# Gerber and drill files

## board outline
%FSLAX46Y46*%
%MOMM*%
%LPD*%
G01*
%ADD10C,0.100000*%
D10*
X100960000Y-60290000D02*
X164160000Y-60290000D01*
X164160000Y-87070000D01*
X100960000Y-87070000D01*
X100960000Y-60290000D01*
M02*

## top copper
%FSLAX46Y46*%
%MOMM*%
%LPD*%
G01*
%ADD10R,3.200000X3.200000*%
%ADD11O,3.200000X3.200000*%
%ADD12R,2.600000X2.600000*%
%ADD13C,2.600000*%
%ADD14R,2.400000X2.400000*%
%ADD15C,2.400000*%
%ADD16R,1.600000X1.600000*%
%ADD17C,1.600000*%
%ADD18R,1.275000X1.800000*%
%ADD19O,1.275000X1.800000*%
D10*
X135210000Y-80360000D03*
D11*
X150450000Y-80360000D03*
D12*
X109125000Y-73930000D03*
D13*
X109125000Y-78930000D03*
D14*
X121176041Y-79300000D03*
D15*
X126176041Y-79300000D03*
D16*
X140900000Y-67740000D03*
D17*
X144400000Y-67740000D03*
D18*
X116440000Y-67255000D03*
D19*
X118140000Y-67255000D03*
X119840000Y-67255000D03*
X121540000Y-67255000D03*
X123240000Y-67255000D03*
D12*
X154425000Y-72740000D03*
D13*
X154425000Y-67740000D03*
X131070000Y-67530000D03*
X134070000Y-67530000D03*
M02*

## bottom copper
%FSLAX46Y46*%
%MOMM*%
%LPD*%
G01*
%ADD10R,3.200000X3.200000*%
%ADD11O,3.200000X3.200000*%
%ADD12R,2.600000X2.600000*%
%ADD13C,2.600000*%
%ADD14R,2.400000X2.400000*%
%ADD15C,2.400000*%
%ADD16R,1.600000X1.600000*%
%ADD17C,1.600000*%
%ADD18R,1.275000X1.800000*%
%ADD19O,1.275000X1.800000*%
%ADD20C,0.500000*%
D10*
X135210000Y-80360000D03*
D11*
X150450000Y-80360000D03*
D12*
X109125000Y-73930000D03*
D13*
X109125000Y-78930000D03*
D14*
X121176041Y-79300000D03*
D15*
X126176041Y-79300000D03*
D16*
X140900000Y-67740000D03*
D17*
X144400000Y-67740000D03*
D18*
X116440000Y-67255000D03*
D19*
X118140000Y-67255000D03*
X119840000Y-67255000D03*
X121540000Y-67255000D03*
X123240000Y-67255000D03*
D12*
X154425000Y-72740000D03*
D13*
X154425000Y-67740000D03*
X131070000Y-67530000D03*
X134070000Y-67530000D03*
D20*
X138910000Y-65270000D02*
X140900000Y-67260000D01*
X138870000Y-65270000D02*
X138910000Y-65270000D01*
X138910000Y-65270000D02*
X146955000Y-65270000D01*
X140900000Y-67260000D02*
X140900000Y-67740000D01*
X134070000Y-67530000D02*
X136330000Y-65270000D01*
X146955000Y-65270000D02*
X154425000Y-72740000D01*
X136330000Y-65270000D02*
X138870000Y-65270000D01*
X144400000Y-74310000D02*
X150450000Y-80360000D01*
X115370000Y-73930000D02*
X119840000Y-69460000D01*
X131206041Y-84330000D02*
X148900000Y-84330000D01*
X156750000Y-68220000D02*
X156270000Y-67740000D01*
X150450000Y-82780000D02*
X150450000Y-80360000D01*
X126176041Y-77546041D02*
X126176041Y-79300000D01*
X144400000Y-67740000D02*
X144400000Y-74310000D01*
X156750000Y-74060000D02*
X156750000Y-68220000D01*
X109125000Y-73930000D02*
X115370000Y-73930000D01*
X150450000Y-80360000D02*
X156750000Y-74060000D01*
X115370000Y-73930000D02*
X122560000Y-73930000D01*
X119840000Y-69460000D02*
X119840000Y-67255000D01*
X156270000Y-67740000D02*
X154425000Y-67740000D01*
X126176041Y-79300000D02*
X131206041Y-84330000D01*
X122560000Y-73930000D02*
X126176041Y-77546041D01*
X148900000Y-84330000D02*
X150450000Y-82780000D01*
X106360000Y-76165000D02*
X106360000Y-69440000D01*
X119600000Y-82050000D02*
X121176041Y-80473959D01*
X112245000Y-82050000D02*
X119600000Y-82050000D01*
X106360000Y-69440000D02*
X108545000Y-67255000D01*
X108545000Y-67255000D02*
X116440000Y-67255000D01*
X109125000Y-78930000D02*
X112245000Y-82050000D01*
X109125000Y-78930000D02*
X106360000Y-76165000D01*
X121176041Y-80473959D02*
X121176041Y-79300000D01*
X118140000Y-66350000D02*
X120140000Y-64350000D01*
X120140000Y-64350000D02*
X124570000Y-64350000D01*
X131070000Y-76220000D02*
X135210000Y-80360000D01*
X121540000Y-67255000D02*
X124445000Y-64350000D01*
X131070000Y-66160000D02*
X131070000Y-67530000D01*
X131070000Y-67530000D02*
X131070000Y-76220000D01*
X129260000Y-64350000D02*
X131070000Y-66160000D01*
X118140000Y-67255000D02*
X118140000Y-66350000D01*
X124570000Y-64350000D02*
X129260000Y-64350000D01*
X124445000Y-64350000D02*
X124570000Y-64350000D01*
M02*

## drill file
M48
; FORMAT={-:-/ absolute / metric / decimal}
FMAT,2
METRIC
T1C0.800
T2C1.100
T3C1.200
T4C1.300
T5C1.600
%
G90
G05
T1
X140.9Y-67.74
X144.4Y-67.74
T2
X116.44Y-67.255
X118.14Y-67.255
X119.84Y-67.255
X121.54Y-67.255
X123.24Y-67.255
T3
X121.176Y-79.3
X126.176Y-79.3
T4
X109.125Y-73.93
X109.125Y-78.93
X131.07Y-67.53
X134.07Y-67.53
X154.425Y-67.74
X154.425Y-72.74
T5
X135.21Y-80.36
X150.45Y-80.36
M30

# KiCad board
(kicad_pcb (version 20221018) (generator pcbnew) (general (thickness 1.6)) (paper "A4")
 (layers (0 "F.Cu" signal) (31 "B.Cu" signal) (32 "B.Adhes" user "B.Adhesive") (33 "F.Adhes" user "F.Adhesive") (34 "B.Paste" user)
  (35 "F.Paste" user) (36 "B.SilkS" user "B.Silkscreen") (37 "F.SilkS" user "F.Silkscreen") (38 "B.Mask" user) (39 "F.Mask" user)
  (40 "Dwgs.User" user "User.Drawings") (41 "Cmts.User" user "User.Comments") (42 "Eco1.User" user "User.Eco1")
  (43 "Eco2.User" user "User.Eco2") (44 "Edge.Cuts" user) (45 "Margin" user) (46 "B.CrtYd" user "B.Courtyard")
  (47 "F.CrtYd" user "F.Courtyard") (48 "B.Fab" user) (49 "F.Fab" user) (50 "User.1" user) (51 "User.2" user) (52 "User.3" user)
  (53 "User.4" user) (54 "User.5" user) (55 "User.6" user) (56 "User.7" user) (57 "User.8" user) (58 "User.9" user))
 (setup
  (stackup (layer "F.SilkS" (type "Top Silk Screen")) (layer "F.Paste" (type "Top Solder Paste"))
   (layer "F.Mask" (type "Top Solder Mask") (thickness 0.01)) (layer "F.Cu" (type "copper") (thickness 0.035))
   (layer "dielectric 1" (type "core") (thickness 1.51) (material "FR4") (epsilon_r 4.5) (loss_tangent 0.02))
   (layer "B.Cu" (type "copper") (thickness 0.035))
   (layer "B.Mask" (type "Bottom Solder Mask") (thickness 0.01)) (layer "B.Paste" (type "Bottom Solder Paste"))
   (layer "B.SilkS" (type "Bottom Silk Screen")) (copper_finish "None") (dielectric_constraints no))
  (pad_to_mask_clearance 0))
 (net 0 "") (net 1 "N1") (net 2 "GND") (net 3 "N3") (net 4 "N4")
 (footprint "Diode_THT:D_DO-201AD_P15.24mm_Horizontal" (layer "F.Cu") (at 135.21 80.36)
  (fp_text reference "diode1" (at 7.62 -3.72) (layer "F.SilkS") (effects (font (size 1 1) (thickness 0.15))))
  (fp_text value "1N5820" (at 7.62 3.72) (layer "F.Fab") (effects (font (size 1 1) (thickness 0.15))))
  (pad "1" thru_hole rect (at 0 0) (size 3.2 3.2) (drill 1.6) (layers "*.Cu" "*.Mask") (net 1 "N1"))
  (pad "2" thru_hole oval (at 15.24 0) (size 3.2 3.2) (drill 1.6) (layers "*.Cu" "*.Mask") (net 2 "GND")))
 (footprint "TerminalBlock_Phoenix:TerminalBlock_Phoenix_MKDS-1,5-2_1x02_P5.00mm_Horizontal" (layer "F.Cu") (at 109.125 73.93 -90)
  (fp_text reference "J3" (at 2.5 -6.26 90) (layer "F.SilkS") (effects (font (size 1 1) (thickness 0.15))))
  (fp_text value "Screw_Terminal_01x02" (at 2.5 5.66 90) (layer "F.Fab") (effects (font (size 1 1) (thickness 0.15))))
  (pad "1" thru_hole rect (at 0 0 270) (size 2.6 2.6) (drill 1.3) (layers "*.Cu" "*.Mask") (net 2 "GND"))
  (pad "2" thru_hole circle (at 5 0 270) (size 2.6 2.6) (drill 1.3) (layers "*.Cu" "*.Mask") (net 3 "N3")))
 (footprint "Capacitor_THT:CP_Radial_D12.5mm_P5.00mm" (layer "F.Cu") (at 121.176041 79.3)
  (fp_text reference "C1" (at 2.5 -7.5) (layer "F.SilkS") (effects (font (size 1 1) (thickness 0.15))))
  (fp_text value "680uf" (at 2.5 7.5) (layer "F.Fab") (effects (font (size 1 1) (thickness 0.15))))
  (pad "1" thru_hole rect (at 0 0) (size 2.4 2.4) (drill 1.2) (layers "*.Cu" "*.Mask") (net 3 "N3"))
  (pad "2" thru_hole circle (at 5 0) (size 2.4 2.4) (drill 1.2) (layers "*.Cu" "*.Mask") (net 2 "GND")))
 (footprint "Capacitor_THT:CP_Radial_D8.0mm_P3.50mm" (layer "F.Cu") (at 140.9 67.74)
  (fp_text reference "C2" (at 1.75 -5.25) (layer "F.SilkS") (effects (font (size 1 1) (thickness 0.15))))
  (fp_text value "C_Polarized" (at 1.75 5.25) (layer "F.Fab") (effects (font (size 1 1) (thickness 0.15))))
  (pad "1" thru_hole rect (at 0 0) (size 1.6 1.6) (drill 0.8) (layers "*.Cu" "*.Mask") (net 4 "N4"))
  (pad "2" thru_hole circle (at 3.5 0) (size 1.6 1.6) (drill 0.8) (layers "*.Cu" "*.Mask") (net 2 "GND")))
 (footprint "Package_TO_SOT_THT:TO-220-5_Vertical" (layer "F.Cu") (at 116.44 67.255)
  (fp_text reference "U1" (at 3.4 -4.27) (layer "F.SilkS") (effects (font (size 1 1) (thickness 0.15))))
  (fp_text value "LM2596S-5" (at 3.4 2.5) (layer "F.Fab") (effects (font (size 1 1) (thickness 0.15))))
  (pad "1" thru_hole rect (at 0 0) (size 1.275 1.8) (drill 1.1) (layers "*.Cu" "*.Mask") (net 3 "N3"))
  (pad "2" thru_hole oval (at 1.7 0) (size 1.275 1.8) (drill 1.1) (layers "*.Cu" "*.Mask") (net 1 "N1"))
  (pad "3" thru_hole oval (at 3.4 0) (size 1.275 1.8) (drill 1.1) (layers "*.Cu" "*.Mask") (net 2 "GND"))
  (pad "4" thru_hole oval (at 5.1 0) (size 1.275 1.8) (drill 1.1) (layers "*.Cu" "*.Mask") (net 1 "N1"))
  (pad "5" thru_hole oval (at 6.8 0) (size 1.275 1.8) (drill 1.1) (layers "*.Cu" "*.Mask") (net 2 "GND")))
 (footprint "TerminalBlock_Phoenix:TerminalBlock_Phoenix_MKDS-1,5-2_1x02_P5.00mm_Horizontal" (layer "F.Cu") (at 154.425 72.74 90)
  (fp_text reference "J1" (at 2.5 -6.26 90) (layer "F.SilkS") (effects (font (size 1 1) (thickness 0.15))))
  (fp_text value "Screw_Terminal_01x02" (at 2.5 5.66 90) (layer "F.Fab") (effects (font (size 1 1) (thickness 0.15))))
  (pad "1" thru_hole rect (at 0 0 90) (size 2.6 2.6) (drill 1.3) (layers "*.Cu" "*.Mask") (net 4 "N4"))
  (pad "2" thru_hole circle (at 5 0 90) (size 2.6 2.6) (drill 1.3) (layers "*.Cu" "*.Mask") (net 2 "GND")))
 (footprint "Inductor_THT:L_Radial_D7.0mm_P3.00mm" (layer "F.Cu") (at 131.07 67.53)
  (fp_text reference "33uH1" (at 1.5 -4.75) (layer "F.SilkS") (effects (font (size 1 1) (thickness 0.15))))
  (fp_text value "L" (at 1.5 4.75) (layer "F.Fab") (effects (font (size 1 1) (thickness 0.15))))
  (pad "1" thru_hole circle (at 0 0) (size 2.6 2.6) (drill 1.3) (layers "*.Cu" "*.Mask") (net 1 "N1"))
  (pad "2" thru_hole circle (at 3 0) (size 2.6 2.6) (drill 1.3) (layers "*.Cu" "*.Mask") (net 4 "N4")))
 (gr_rect (start 100.96 60.29) (end 164.16 87.07) (stroke (width 0.1) (type default)) (fill none) (layer "Edge.Cuts"))
 (segment (start 138.91 65.27) (end 140.9 67.26) (width 0.5) (layer "B.Cu") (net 4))
 (segment (start 138.87 65.27) (end 138.91 65.27) (width 0.5) (layer "B.Cu") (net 4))
 (segment (start 138.91 65.27) (end 146.955 65.27) (width 0.5) (layer "B.Cu") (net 4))
 (segment (start 140.9 67.26) (end 140.9 67.74) (width 0.5) (layer "B.Cu") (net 4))
 (segment (start 134.07 67.53) (end 136.33 65.27) (width 0.5) (layer "B.Cu") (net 4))
 (segment (start 146.955 65.27) (end 154.425 72.74) (width 0.5) (layer "B.Cu") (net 4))
 (segment (start 136.33 65.27) (end 138.87 65.27) (width 0.5) (layer "B.Cu") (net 4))
 (segment (start 144.4 74.31) (end 150.45 80.36) (width 0.5) (layer "B.Cu") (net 2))
 (segment (start 115.37 73.93) (end 119.84 69.46) (width 0.5) (layer "B.Cu") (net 2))
 (segment (start 131.206041 84.33) (end 148.9 84.33) (width 0.5) (layer "B.Cu") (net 2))
 (segment (start 156.75 68.22) (end 156.27 67.74) (width 0.5) (layer "B.Cu") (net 2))
 (segment (start 150.45 82.78) (end 150.45 80.36) (width 0.5) (layer "B.Cu") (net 2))
 (segment (start 126.176041 77.546041) (end 126.176041 79.3) (width 0.5) (layer "B.Cu") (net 2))
 (segment (start 144.4 67.74) (end 144.4 74.31) (width 0.5) (layer "B.Cu") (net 2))
 (segment (start 156.75 74.06) (end 156.75 68.22) (width 0.5) (layer "B.Cu") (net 2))
 (segment (start 109.125 73.93) (end 115.37 73.93) (width 0.5) (layer "B.Cu") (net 2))
 (segment (start 150.45 80.36) (end 156.75 74.06) (width 0.5) (layer "B.Cu") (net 2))
 (segment (start 115.37 73.93) (end 122.56 73.93) (width 0.5) (layer "B.Cu") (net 2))
 (segment (start 119.84 69.46) (end 119.84 67.255) (width 0.5) (layer "B.Cu") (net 2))
 (segment (start 156.27 67.74) (end 154.425 67.74) (width 0.5) (layer "B.Cu") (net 2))
 (segment (start 126.176041 79.3) (end 131.206041 84.33) (width 0.5) (layer "B.Cu") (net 2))
 (segment (start 122.56 73.93) (end 126.176041 77.546041) (width 0.5) (layer "B.Cu") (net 2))
 (segment (start 148.9 84.33) (end 150.45 82.78) (width 0.5) (layer "B.Cu") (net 2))
 (segment (start 106.36 76.165) (end 106.36 69.44) (width 0.5) (layer "B.Cu") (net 3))
 (segment (start 119.6 82.05) (end 121.176041 80.473959) (width 0.5) (layer "B.Cu") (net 3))
 (segment (start 112.245 82.05) (end 119.6 82.05) (width 0.5) (layer "B.Cu") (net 3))
 (segment (start 106.36 69.44) (end 108.545 67.255) (width 0.5) (layer "B.Cu") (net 3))
 (segment (start 108.545 67.255) (end 116.44 67.255) (width 0.5) (layer "B.Cu") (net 3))
 (segment (start 109.125 78.93) (end 112.245 82.05) (width 0.5) (layer "B.Cu") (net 3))
 (segment (start 109.125 78.93) (end 106.36 76.165) (width 0.5) (layer "B.Cu") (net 3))
 (segment (start 121.176041 80.473959) (end 121.176041 79.3) (width 0.5) (layer "B.Cu") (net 3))
 (segment (start 118.14 66.35) (end 120.14 64.35) (width 0.5) (layer "B.Cu") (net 1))
 (segment (start 120.14 64.35) (end 124.57 64.35) (width 0.5) (layer "B.Cu") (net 1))
 (segment (start 131.07 76.22) (end 135.21 80.36) (width 0.5) (layer "B.Cu") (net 1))
 (segment (start 121.54 67.255) (end 124.445 64.35) (width 0.5) (layer "B.Cu") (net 1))
 (segment (start 131.07 66.16) (end 131.07 67.53) (width 0.5) (layer "B.Cu") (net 1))
 (segment (start 131.07 67.53) (end 131.07 76.22) (width 0.5) (layer "B.Cu") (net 1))
 (segment (start 129.26 64.35) (end 131.07 66.16) (width 0.5) (layer "B.Cu") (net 1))
 (segment (start 118.14 67.255) (end 118.14 66.35) (width 0.5) (layer "B.Cu") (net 1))
 (segment (start 124.57 64.35) (end 129.26 64.35) (width 0.5) (layer "B.Cu") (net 1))
 (segment (start 124.445 64.35) (end 124.57 64.35) (width 0.5) (layer "B.Cu") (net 1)))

